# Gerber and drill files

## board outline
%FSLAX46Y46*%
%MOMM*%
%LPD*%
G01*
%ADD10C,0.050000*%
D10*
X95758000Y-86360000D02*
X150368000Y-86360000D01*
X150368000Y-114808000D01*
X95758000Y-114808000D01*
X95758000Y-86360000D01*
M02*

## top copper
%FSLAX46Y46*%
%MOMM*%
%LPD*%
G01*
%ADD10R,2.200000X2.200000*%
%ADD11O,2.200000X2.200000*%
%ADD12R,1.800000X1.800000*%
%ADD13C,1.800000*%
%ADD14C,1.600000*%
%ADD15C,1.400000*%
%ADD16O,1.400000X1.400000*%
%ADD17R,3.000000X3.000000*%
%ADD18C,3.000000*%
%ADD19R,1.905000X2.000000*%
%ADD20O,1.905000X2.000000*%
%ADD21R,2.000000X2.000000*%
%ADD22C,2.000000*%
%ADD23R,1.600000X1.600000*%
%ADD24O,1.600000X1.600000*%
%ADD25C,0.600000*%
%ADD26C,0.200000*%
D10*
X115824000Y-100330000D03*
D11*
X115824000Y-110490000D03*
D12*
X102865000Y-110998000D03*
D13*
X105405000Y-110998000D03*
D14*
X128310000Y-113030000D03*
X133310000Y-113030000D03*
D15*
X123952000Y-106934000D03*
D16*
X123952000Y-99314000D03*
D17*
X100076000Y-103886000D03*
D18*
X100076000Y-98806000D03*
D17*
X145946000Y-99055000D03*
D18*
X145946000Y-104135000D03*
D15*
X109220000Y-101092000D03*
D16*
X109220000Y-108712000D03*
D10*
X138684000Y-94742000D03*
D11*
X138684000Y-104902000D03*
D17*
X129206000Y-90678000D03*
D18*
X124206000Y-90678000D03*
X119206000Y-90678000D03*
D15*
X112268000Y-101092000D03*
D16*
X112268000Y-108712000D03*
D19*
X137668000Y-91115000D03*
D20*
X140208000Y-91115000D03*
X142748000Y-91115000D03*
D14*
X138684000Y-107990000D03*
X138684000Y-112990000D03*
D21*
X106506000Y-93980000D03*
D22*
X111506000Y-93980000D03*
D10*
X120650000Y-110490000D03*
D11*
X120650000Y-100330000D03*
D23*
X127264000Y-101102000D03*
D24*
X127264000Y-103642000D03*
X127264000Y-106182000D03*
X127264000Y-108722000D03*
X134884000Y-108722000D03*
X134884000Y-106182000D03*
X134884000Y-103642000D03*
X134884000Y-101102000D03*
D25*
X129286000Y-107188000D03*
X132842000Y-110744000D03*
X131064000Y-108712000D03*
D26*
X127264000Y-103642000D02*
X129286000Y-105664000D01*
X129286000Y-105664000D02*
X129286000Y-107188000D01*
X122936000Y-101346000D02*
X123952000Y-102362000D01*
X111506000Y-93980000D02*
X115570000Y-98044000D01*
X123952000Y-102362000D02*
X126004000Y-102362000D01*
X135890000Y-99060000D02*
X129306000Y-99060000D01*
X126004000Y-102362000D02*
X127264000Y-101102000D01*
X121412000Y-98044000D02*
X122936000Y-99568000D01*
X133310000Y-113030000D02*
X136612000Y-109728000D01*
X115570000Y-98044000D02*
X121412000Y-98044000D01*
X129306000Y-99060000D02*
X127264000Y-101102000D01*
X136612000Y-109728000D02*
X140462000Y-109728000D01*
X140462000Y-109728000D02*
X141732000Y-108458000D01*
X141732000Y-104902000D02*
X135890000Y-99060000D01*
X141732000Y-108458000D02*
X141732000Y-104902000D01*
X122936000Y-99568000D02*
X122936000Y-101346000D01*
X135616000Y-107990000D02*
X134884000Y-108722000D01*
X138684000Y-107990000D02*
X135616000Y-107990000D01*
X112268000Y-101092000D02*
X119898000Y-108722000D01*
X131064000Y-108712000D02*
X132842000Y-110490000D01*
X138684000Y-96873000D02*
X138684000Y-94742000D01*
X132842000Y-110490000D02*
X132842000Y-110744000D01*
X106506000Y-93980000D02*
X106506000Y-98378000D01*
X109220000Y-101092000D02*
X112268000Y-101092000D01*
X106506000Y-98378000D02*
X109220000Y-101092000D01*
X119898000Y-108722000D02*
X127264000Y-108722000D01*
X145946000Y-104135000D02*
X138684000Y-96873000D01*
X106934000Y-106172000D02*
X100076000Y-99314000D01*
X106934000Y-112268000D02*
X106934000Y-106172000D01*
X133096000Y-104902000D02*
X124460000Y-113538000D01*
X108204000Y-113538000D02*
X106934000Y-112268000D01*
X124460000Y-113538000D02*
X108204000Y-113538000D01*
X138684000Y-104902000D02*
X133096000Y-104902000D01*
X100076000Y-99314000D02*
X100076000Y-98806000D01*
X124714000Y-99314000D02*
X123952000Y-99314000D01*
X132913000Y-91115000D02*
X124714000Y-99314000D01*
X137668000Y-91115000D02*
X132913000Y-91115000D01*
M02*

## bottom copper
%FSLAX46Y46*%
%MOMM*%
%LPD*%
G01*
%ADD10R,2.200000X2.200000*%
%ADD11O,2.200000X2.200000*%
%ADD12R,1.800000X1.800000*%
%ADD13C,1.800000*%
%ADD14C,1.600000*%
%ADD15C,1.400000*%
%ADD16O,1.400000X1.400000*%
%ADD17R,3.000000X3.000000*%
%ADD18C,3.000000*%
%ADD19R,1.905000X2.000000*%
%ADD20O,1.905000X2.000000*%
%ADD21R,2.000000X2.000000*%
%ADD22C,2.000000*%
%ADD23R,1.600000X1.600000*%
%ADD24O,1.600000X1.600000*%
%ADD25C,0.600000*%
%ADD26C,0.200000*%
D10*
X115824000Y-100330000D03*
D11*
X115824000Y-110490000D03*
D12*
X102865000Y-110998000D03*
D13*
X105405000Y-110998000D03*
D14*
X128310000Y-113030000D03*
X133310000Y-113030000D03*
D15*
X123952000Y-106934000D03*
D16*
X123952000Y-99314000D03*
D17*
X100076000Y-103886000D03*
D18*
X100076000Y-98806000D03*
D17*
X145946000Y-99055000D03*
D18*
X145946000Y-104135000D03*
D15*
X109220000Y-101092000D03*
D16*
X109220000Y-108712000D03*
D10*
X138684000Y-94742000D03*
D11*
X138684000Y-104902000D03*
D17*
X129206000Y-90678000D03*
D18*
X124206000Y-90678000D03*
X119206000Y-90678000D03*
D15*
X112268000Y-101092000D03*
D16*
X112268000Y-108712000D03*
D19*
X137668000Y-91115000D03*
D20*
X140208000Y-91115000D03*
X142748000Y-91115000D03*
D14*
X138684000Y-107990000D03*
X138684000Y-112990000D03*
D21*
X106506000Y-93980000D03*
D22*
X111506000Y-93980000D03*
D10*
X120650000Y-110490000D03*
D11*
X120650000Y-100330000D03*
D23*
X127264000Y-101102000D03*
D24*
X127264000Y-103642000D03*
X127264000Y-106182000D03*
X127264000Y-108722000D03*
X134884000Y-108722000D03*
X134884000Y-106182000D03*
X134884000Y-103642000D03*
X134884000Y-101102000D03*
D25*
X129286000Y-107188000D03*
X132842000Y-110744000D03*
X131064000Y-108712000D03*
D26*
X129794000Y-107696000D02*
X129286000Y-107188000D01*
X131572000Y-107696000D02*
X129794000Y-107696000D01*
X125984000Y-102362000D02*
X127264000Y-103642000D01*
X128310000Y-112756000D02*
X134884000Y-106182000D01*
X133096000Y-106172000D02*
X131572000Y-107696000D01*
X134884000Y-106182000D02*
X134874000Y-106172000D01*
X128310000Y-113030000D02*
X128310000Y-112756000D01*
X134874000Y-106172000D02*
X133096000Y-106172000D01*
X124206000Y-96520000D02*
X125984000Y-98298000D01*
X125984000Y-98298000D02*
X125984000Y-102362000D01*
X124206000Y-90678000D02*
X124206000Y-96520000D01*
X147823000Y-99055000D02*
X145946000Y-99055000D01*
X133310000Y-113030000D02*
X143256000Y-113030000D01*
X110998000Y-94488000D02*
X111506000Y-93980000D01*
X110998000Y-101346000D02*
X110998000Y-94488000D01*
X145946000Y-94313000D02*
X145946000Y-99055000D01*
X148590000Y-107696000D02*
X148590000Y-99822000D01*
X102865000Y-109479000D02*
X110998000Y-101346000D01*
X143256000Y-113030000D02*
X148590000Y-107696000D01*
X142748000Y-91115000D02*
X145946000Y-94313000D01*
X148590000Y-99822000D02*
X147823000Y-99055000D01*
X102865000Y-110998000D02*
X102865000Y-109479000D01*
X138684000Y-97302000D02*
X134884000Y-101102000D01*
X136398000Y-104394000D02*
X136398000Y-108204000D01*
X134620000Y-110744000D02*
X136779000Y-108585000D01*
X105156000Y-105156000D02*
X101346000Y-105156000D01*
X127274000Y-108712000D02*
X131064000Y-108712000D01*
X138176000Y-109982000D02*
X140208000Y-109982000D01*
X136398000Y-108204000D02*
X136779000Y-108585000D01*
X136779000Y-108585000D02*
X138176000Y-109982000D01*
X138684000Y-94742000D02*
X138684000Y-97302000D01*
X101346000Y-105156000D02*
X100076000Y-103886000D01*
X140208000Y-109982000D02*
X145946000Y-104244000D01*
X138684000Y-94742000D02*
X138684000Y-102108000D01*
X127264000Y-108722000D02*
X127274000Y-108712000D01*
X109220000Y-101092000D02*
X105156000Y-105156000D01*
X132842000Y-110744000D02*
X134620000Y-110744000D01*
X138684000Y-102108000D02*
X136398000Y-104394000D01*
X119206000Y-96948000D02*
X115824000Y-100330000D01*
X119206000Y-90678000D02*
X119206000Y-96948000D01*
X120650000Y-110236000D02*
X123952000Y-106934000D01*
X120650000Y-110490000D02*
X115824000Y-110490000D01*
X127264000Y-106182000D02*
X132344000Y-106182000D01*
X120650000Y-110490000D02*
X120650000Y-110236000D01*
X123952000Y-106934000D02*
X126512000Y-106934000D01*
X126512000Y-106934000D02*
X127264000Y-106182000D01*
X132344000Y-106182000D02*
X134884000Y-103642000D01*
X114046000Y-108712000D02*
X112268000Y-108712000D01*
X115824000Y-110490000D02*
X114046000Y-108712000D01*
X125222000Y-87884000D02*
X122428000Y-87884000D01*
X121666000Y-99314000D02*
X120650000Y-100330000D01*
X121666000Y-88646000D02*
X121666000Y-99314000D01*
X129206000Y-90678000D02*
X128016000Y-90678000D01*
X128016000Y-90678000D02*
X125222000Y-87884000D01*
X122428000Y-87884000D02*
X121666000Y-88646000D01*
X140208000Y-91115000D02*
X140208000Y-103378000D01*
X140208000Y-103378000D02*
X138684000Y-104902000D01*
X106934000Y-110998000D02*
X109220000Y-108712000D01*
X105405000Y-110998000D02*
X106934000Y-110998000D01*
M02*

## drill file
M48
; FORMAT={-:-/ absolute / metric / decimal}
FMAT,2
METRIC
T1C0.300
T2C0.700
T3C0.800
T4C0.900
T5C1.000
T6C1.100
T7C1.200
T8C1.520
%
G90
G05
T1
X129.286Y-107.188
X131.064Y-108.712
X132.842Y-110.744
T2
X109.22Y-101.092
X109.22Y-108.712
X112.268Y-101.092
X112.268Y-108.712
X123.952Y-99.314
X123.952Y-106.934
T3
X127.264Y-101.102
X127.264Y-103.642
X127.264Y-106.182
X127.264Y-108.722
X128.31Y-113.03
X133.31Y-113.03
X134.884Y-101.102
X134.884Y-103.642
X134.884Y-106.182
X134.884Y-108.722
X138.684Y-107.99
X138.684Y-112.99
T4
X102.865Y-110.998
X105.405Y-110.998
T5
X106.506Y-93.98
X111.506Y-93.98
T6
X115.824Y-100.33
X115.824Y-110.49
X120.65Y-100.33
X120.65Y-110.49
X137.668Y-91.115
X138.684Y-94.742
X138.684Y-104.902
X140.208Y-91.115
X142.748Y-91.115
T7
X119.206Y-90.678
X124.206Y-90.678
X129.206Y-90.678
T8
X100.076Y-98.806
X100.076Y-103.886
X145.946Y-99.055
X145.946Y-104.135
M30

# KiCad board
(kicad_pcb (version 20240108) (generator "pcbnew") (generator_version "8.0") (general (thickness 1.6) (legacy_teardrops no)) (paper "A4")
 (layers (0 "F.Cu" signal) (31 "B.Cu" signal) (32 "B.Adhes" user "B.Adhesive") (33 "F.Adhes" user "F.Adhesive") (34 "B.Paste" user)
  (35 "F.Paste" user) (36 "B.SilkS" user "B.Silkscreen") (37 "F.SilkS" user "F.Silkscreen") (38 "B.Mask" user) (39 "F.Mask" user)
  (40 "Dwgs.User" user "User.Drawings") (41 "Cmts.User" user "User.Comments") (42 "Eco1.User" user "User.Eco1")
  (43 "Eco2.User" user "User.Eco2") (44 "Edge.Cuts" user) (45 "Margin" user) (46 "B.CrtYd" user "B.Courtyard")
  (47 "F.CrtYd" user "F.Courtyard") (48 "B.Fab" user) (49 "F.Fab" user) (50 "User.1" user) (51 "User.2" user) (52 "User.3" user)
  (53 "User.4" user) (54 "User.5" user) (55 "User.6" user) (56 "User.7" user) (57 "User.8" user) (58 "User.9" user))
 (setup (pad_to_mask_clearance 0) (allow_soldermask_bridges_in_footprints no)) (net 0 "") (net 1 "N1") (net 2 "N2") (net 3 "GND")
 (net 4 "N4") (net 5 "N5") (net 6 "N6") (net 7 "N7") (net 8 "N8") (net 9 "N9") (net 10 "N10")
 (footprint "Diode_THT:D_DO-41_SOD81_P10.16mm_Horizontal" (layer "F.Cu") (at 115.824 100.33 -90)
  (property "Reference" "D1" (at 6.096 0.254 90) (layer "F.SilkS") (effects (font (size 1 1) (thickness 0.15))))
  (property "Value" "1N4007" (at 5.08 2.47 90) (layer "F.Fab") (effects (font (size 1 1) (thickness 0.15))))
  (pad "1" thru_hole rect (at 0 0 270) (size 2.2 2.2) (drill 1.1) (layers "*.Cu" "*.Mask") (remove_unused_layers no) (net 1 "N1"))
  (pad "2" thru_hole oval (at 10.16 0 270) (size 2.2 2.2) (drill 1.1) (layers "*.Cu" "*.Mask") (remove_unused_layers no) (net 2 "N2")))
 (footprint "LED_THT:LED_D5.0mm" (layer "F.Cu") (at 102.865 110.998)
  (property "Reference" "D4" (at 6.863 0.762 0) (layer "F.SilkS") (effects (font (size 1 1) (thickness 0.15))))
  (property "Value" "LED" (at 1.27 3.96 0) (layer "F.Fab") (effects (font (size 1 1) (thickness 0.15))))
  (pad "1" thru_hole rect (at 0 0) (size 1.8 1.8) (drill 0.9) (layers "*.Cu" "*.Mask") (remove_unused_layers no) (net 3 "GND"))
  (pad "2" thru_hole circle (at 2.54 0) (size 1.8 1.8) (drill 0.9) (layers "*.Cu" "*.Mask") (remove_unused_layers no) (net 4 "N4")))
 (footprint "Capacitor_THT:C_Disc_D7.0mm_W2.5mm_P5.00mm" (layer "F.Cu") (at 128.31 113.03)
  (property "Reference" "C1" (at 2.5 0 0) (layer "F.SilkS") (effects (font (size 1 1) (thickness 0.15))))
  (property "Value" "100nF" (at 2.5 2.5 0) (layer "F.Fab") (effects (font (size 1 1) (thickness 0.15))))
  (pad "1" thru_hole circle (at 0 0) (size 1.6 1.6) (drill 0.8) (layers "*.Cu" "*.Mask") (remove_unused_layers no) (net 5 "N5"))
  (pad "2" thru_hole circle (at 5 0) (size 1.6 1.6) (drill 0.8) (layers "*.Cu" "*.Mask") (remove_unused_layers no) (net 3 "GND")))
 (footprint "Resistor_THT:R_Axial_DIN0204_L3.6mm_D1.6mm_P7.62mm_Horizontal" (layer "F.Cu") (at 123.952 106.934 90)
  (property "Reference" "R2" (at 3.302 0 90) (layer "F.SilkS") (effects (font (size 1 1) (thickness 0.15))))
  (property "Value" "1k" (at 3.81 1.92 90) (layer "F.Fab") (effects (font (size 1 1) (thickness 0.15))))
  (pad "1" thru_hole circle (at 0 0 90) (size 1.4 1.4) (drill 0.7) (layers "*.Cu" "*.Mask") (remove_unused_layers no) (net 2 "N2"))
  (pad "2" thru_hole oval (at 7.62 0 90) (size 1.4 1.4) (drill 0.7) (layers "*.Cu" "*.Mask") (remove_unused_layers no) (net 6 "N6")))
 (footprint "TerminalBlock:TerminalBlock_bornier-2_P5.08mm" (layer "F.Cu") (at 100.076 103.886 90)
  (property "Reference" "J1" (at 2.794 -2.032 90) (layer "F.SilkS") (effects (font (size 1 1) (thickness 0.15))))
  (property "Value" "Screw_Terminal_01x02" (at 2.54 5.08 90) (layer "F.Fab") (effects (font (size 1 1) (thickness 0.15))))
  (pad "1" thru_hole rect (at 0 0 90) (size 3 3) (drill 1.52) (layers "*.Cu" "*.Mask") (remove_unused_layers no) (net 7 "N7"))
  (pad "2" thru_hole circle (at 5.08 0 90) (size 3 3) (drill 1.52) (layers "*.Cu" "*.Mask") (remove_unused_layers no) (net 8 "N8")))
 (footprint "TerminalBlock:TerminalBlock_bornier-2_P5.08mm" (layer "F.Cu") (at 145.946 99.055 -90)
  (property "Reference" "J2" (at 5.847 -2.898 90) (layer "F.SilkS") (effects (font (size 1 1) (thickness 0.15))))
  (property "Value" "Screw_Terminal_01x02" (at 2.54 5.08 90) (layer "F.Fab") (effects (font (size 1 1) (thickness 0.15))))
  (pad "1" thru_hole rect (at 0 0 270) (size 3 3) (drill 1.52) (layers "*.Cu" "*.Mask") (remove_unused_layers no) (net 3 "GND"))
  (pad "2" thru_hole circle (at 5.08 0 270) (size 3 3) (drill 1.52) (layers "*.Cu" "*.Mask") (remove_unused_layers no) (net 7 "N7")))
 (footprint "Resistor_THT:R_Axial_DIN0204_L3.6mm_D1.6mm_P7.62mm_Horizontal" (layer "F.Cu") (at 109.22 101.092 -90)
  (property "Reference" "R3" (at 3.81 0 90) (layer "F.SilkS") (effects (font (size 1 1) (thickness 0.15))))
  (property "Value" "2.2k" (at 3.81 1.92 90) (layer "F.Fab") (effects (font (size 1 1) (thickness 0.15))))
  (pad "1" thru_hole circle (at 0 0 270) (size 1.4 1.4) (drill 0.7) (layers "*.Cu" "*.Mask") (remove_unused_layers no) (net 7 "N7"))
  (pad "2" thru_hole oval (at 7.62 0 270) (size 1.4 1.4) (drill 0.7) (layers "*.Cu" "*.Mask") (remove_unused_layers no) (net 4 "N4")))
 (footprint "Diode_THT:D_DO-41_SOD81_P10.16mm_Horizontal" (layer "F.Cu") (at 138.684 94.742 -90)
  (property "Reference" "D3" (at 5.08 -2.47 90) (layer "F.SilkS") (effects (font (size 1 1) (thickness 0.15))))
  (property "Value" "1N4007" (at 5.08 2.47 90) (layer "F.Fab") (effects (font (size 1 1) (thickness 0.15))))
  (pad "1" thru_hole rect (at 0 0 270) (size 2.2 2.2) (drill 1.1) (layers "*.Cu" "*.Mask") (remove_unused_layers no) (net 7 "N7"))
  (pad "2" thru_hole oval (at 10.16 0 270) (size 2.2 2.2) (drill 1.1) (layers "*.Cu" "*.Mask") (remove_unused_layers no) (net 8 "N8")))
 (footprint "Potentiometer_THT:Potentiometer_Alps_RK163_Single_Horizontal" (layer "F.Cu") (at 129.206 90.678 -90)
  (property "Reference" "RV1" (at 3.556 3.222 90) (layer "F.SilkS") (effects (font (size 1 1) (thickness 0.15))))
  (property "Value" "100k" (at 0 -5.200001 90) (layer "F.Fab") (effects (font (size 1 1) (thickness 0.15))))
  (pad "1" thru_hole rect (at 0 0 90) (size 3 3) (drill 1.2) (layers "*.Cu" "*.Mask") (remove_unused_layers no) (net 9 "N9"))
  (pad "2" thru_hole circle (at 0 5 90) (size 3 3) (drill 1.2) (layers "*.Cu" "*.Mask") (remove_unused_layers no) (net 5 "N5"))
  (pad "3" thru_hole circle (at 0 10 90) (size 3 3) (drill 1.2) (layers "*.Cu" "*.Mask") (remove_unused_layers no) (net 1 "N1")))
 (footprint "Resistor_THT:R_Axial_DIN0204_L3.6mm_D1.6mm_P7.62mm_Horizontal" (layer "F.Cu") (at 112.268 101.092 -90)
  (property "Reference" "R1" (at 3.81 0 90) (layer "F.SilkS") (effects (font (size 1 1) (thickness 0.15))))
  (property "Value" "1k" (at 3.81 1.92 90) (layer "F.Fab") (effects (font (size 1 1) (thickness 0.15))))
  (pad "1" thru_hole circle (at 0 0 270) (size 1.4 1.4) (drill 0.7) (layers "*.Cu" "*.Mask") (remove_unused_layers no) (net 7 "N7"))
  (pad "2" thru_hole oval (at 7.62 0 270) (size 1.4 1.4) (drill 0.7) (layers "*.Cu" "*.Mask") (remove_unused_layers no) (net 2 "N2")))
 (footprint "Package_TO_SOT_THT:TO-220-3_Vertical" (layer "F.Cu") (at 137.668 91.115)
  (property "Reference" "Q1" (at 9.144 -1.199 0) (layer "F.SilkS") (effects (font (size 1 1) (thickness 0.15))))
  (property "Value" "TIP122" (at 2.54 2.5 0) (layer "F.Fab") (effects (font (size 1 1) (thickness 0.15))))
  (pad "1" thru_hole rect (at 0 0) (size 1.905 2) (drill 1.1) (layers "*.Cu" "*.Mask") (remove_unused_layers no) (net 6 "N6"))
  (pad "2" thru_hole oval (at 2.54 0) (size 1.905 2) (drill 1.1) (layers "*.Cu" "*.Mask") (remove_unused_layers no) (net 8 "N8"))
  (pad "3" thru_hole oval (at 5.08 0) (size 1.905 2) (drill 1.1) (layers "*.Cu" "*.Mask") (remove_unused_layers no) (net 3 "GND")))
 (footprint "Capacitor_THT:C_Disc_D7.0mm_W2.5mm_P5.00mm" (layer "F.Cu") (at 138.684 107.99 -90)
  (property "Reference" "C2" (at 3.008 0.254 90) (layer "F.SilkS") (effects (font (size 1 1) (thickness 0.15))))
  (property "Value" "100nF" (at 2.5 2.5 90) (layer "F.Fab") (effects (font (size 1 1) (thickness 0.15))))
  (pad "1" thru_hole circle (at 0 0 270) (size 1.6 1.6) (drill 0.8) (layers "*.Cu" "*.Mask") (remove_unused_layers no) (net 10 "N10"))
  (pad "2" thru_hole circle (at 5 0 270) (size 1.6 1.6) (drill 0.8) (layers "*.Cu" "*.Mask") (remove_unused_layers no) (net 3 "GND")))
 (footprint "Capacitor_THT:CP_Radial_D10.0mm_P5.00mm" (layer "F.Cu") (at 106.506 93.98)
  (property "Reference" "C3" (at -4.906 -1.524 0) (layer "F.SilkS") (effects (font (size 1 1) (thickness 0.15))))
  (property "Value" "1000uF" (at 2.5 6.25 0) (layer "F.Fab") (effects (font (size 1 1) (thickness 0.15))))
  (pad "1" thru_hole rect (at 0 0) (size 2 2) (drill 1) (layers "*.Cu" "*.Mask") (remove_unused_layers no) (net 7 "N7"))
  (pad "2" thru_hole circle (at 5 0) (size 2 2) (drill 1) (layers "*.Cu" "*.Mask") (remove_unused_layers no) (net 3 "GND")))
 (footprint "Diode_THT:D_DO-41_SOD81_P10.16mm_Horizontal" (layer "F.Cu") (at 120.65 110.49 90)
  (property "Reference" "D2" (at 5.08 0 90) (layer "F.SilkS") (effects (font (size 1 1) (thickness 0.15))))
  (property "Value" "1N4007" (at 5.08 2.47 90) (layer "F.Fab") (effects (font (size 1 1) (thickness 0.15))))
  (pad "1" thru_hole rect (at 0 0 90) (size 2.2 2.2) (drill 1.1) (layers "*.Cu" "*.Mask") (remove_unused_layers no) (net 2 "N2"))
  (pad "2" thru_hole oval (at 10.16 0 90) (size 2.2 2.2) (drill 1.1) (layers "*.Cu" "*.Mask") (remove_unused_layers no) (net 9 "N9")))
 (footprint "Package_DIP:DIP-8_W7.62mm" (layer "F.Cu") (at 127.264 101.102)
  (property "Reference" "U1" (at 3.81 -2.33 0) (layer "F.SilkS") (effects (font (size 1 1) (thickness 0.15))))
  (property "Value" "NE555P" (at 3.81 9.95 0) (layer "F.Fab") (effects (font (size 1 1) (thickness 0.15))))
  (pad "1" thru_hole rect (at 0 0) (size 1.6 1.6) (drill 0.8) (layers "*.Cu" "*.Mask") (remove_unused_layers no) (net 3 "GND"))
  (pad "2" thru_hole oval (at 0 2.54) (size 1.6 1.6) (drill 0.8) (layers "*.Cu" "*.Mask") (remove_unused_layers no) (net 5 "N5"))
  (pad "3" thru_hole oval (at 0 5.08) (size 1.6 1.6) (drill 0.8) (layers "*.Cu" "*.Mask") (remove_unused_layers no) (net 2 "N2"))
  (pad "4" thru_hole oval (at 0 7.62) (size 1.6 1.6) (drill 0.8) (layers "*.Cu" "*.Mask") (remove_unused_layers no) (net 7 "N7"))
  (pad "5" thru_hole oval (at 7.62 7.62) (size 1.6 1.6) (drill 0.8) (layers "*.Cu" "*.Mask") (remove_unused_layers no) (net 10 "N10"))
  (pad "6" thru_hole oval (at 7.62 5.08) (size 1.6 1.6) (drill 0.8) (layers "*.Cu" "*.Mask") (remove_unused_layers no) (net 5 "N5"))
  (pad "7" thru_hole oval (at 7.62 2.54) (size 1.6 1.6) (drill 0.8) (layers "*.Cu" "*.Mask") (remove_unused_layers no) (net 2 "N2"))
  (pad "8" thru_hole oval (at 7.62 0) (size 1.6 1.6) (drill 0.8) (layers "*.Cu" "*.Mask") (remove_unused_layers no) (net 7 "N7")))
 (gr_rect (start 95.758 86.36) (end 150.368 114.808) (stroke (width 0.05) (type default)) (fill none) (layer "Edge.Cuts"))
 (segment (start 127.264 103.642) (end 129.286 105.664) (width 0.2) (layer "F.Cu") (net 5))
 (segment (start 129.286 105.664) (end 129.286 107.188) (width 0.2) (layer "F.Cu") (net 5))
 (via (at 129.286 107.188) (size 0.6) (drill 0.3) (layers "F.Cu" "B.Cu") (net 5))
 (segment (start 129.794 107.696) (end 129.286 107.188) (width 0.2) (layer "B.Cu") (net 5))
 (segment (start 131.572 107.696) (end 129.794 107.696) (width 0.2) (layer "B.Cu") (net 5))
 (segment (start 125.984 102.362) (end 127.264 103.642) (width 0.2) (layer "B.Cu") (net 5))
 (segment (start 128.31 112.756) (end 134.884 106.182) (width 0.2) (layer "B.Cu") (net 5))
 (segment (start 133.096 106.172) (end 131.572 107.696) (width 0.2) (layer "B.Cu") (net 5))
 (segment (start 134.884 106.182) (end 134.874 106.172) (width 0.2) (layer "B.Cu") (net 5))
 (segment (start 128.31 113.03) (end 128.31 112.756) (width 0.2) (layer "B.Cu") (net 5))
 (segment (start 134.874 106.172) (end 133.096 106.172) (width 0.2) (layer "B.Cu") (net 5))
 (segment (start 124.206 96.52) (end 125.984 98.298) (width 0.2) (layer "B.Cu") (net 5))
 (segment (start 125.984 98.298) (end 125.984 102.362) (width 0.2) (layer "B.Cu") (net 5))
 (segment (start 124.206 90.678) (end 124.206 96.52) (width 0.2) (layer "B.Cu") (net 5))
 (segment (start 122.936 101.346) (end 123.952 102.362) (width 0.2) (layer "F.Cu") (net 3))
 (segment (start 111.506 93.98) (end 115.57 98.044) (width 0.2) (layer "F.Cu") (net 3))
 (segment (start 123.952 102.362) (end 126.004 102.362) (width 0.2) (layer "F.Cu") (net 3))
 (segment (start 135.89 99.06) (end 129.306 99.06) (width 0.2) (layer "F.Cu") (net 3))
 (segment (start 126.004 102.362) (end 127.264 101.102) (width 0.2) (layer "F.Cu") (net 3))
 (segment (start 121.412 98.044) (end 122.936 99.568) (width 0.2) (layer "F.Cu") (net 3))
 (segment (start 133.31 113.03) (end 136.612 109.728) (width 0.2) (layer "F.Cu") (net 3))
 (segment (start 115.57 98.044) (end 121.412 98.044) (width 0.2) (layer "F.Cu") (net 3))
 (segment (start 129.306 99.06) (end 127.264 101.102) (width 0.2) (layer "F.Cu") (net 3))
 (segment (start 136.612 109.728) (end 140.462 109.728) (width 0.2) (layer "F.Cu") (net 3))
 (segment (start 140.462 109.728) (end 141.732 108.458) (width 0.2) (layer "F.Cu") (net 3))
 (segment (start 141.732 104.902) (end 135.89 99.06) (width 0.2) (layer "F.Cu") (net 3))
 (segment (start 141.732 108.458) (end 141.732 104.902) (width 0.2) (layer "F.Cu") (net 3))
 (segment (start 122.936 99.568) (end 122.936 101.346) (width 0.2) (layer "F.Cu") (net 3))
 (segment (start 147.823 99.055) (end 145.946 99.055) (width 0.2) (layer "B.Cu") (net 3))
 (segment (start 133.31 113.03) (end 143.256 113.03) (width 0.2) (layer "B.Cu") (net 3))
 (segment (start 110.998 94.488) (end 111.506 93.98) (width 0.2) (layer "B.Cu") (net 3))
 (segment (start 110.998 101.346) (end 110.998 94.488) (width 0.2) (layer "B.Cu") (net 3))
 (segment (start 145.946 94.313) (end 145.946 99.055) (width 0.2) (layer "B.Cu") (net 3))
 (segment (start 148.59 107.696) (end 148.59 99.822) (width 0.2) (layer "B.Cu") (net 3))
 (segment (start 102.865 109.479) (end 110.998 101.346) (width 0.2) (layer "B.Cu") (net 3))
 (segment (start 143.256 113.03) (end 148.59 107.696) (width 0.2) (layer "B.Cu") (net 3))
 (segment (start 142.748 91.115) (end 145.946 94.313) (width 0.2) (layer "B.Cu") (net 3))
 (segment (start 148.59 99.822) (end 147.823 99.055) (width 0.2) (layer "B.Cu") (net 3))
 (segment (start 102.865 110.998) (end 102.865 109.479) (width 0.2) (layer "B.Cu") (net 3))
 (segment (start 135.616 107.99) (end 134.884 108.722) (width 0.2) (layer "F.Cu") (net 10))
 (segment (start 138.684 107.99) (end 135.616 107.99) (width 0.2) (layer "F.Cu") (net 10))
 (segment (start 112.268 101.092) (end 119.898 108.722) (width 0.2) (layer "F.Cu") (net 7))
 (segment (start 131.064 108.712) (end 132.842 110.49) (width 0.2) (layer "F.Cu") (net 7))
 (segment (start 138.684 96.873) (end 138.684 94.742) (width 0.2) (layer "F.Cu") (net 7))
 (segment (start 132.842 110.49) (end 132.842 110.744) (width 0.2) (layer "F.Cu") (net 7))
 (segment (start 106.506 93.98) (end 106.506 98.378) (width 0.2) (layer "F.Cu") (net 7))
 (segment (start 109.22 101.092) (end 112.268 101.092) (width 0.2) (layer "F.Cu") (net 7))
 (segment (start 106.506 98.378) (end 109.22 101.092) (width 0.2) (layer "F.Cu") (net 7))
 (segment (start 119.898 108.722) (end 127.264 108.722) (width 0.2) (layer "F.Cu") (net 7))
 (segment (start 145.946 104.135) (end 138.684 96.873) (width 0.2) (layer "F.Cu") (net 7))
 (via (at 132.842 110.744) (size 0.6) (drill 0.3) (layers "F.Cu" "B.Cu") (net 7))
 (via (at 131.064 108.712) (size 0.6) (drill 0.3) (layers "F.Cu" "B.Cu") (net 7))
 (segment (start 138.684 97.302) (end 134.884 101.102) (width 0.2) (layer "B.Cu") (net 7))
 (segment (start 136.398 104.394) (end 136.398 108.204) (width 0.2) (layer "B.Cu") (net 7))
 (segment (start 134.62 110.744) (end 136.779 108.585) (width 0.2) (layer "B.Cu") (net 7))
 (segment (start 105.156 105.156) (end 101.346 105.156) (width 0.2) (layer "B.Cu") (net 7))
 (segment (start 127.274 108.712) (end 131.064 108.712) (width 0.2) (layer "B.Cu") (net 7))
 (segment (start 138.176 109.982) (end 140.208 109.982) (width 0.2) (layer "B.Cu") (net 7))
 (segment (start 136.398 108.204) (end 136.779 108.585) (width 0.2) (layer "B.Cu") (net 7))
 (segment (start 136.779 108.585) (end 138.176 109.982) (width 0.2) (layer "B.Cu") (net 7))
 (segment (start 138.684 94.742) (end 138.684 97.302) (width 0.2) (layer "B.Cu") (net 7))
 (segment (start 101.346 105.156) (end 100.076 103.886) (width 0.2) (layer "B.Cu") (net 7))
 (segment (start 140.208 109.982) (end 145.946 104.244) (width 0.2) (layer "B.Cu") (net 7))
 (segment (start 138.684 94.742) (end 138.684 102.108) (width 0.2) (layer "B.Cu") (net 7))
 (segment (start 127.264 108.722) (end 127.274 108.712) (width 0.2) (layer "B.Cu") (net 7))
 (segment (start 109.22 101.092) (end 105.156 105.156) (width 0.2) (layer "B.Cu") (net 7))
 (segment (start 132.842 110.744) (end 134.62 110.744) (width 0.2) (layer "B.Cu") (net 7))
 (segment (start 138.684 102.108) (end 136.398 104.394) (width 0.2) (layer "B.Cu") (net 7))
 (segment (start 119.206 96.948) (end 115.824 100.33) (width 0.2) (layer "B.Cu") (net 1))
 (segment (start 119.206 90.678) (end 119.206 96.948) (width 0.2) (layer "B.Cu") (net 1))
 (segment (start 120.65 110.236) (end 123.952 106.934) (width 0.2) (layer "B.Cu") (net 2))
 (segment (start 120.65 110.49) (end 115.824 110.49) (width 0.2) (layer "B.Cu") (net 2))
 (segment (start 127.264 106.182) (end 132.344 106.182) (width 0.2) (layer "B.Cu") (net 2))
 (segment (start 120.65 110.49) (end 120.65 110.236) (width 0.2) (layer "B.Cu") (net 2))
 (segment (start 123.952 106.934) (end 126.512 106.934) (width 0.2) (layer "B.Cu") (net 2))
 (segment (start 126.512 106.934) (end 127.264 106.182) (width 0.2) (layer "B.Cu") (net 2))
 (segment (start 132.344 106.182) (end 134.884 103.642) (width 0.2) (layer "B.Cu") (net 2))
 (segment (start 114.046 108.712) (end 112.268 108.712) (width 0.2) (layer "B.Cu") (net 2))
 (segment (start 115.824 110.49) (end 114.046 108.712) (width 0.2) (layer "B.Cu") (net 2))
 (segment (start 125.222 87.884) (end 122.428 87.884) (width 0.2) (layer "B.Cu") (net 9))
 (segment (start 121.666 99.314) (end 120.65 100.33) (width 0.2) (layer "B.Cu") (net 9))
 (segment (start 121.666 88.646) (end 121.666 99.314) (width 0.2) (layer "B.Cu") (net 9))
 (segment (start 129.206 90.678) (end 128.016 90.678) (width 0.2) (layer "B.Cu") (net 9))
 (segment (start 128.016 90.678) (end 125.222 87.884) (width 0.2) (layer "B.Cu") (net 9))
 (segment (start 122.428 87.884) (end 121.666 88.646) (width 0.2) (layer "B.Cu") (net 9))
 (segment (start 106.934 106.172) (end 100.076 99.314) (width 0.2) (layer "F.Cu") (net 8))
 (segment (start 106.934 112.268) (end 106.934 106.172) (width 0.2) (layer "F.Cu") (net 8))
 (segment (start 133.096 104.902) (end 124.46 113.538) (width 0.2) (layer "F.Cu") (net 8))
 (segment (start 108.204 113.538) (end 106.934 112.268) (width 0.2) (layer "F.Cu") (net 8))
 (segment (start 124.46 113.538) (end 108.204 113.538) (width 0.2) (layer "F.Cu") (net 8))
 (segment (start 138.684 104.902) (end 133.096 104.902) (width 0.2) (layer "F.Cu") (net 8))
 (segment (start 100.076 99.314) (end 100.076 98.806) (width 0.2) (layer "F.Cu") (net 8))
 (segment (start 140.208 91.115) (end 140.208 103.378) (width 0.2) (layer "B.Cu") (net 8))
 (segment (start 140.208 103.378) (end 138.684 104.902) (width 0.2) (layer "B.Cu") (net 8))
 (segment (start 106.934 110.998) (end 109.22 108.712) (width 0.2) (layer "B.Cu") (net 4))
 (segment (start 105.405 110.998) (end 106.934 110.998) (width 0.2) (layer "B.Cu") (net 4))
 (segment (start 124.714 99.314) (end 123.952 99.314) (width 0.2) (layer "F.Cu") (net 6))
 (segment (start 132.913 91.115) (end 124.714 99.314) (width 0.2) (layer "F.Cu") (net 6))
 (segment (start 137.668 91.115) (end 132.913 91.115) (width 0.2) (layer "F.Cu") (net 6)))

